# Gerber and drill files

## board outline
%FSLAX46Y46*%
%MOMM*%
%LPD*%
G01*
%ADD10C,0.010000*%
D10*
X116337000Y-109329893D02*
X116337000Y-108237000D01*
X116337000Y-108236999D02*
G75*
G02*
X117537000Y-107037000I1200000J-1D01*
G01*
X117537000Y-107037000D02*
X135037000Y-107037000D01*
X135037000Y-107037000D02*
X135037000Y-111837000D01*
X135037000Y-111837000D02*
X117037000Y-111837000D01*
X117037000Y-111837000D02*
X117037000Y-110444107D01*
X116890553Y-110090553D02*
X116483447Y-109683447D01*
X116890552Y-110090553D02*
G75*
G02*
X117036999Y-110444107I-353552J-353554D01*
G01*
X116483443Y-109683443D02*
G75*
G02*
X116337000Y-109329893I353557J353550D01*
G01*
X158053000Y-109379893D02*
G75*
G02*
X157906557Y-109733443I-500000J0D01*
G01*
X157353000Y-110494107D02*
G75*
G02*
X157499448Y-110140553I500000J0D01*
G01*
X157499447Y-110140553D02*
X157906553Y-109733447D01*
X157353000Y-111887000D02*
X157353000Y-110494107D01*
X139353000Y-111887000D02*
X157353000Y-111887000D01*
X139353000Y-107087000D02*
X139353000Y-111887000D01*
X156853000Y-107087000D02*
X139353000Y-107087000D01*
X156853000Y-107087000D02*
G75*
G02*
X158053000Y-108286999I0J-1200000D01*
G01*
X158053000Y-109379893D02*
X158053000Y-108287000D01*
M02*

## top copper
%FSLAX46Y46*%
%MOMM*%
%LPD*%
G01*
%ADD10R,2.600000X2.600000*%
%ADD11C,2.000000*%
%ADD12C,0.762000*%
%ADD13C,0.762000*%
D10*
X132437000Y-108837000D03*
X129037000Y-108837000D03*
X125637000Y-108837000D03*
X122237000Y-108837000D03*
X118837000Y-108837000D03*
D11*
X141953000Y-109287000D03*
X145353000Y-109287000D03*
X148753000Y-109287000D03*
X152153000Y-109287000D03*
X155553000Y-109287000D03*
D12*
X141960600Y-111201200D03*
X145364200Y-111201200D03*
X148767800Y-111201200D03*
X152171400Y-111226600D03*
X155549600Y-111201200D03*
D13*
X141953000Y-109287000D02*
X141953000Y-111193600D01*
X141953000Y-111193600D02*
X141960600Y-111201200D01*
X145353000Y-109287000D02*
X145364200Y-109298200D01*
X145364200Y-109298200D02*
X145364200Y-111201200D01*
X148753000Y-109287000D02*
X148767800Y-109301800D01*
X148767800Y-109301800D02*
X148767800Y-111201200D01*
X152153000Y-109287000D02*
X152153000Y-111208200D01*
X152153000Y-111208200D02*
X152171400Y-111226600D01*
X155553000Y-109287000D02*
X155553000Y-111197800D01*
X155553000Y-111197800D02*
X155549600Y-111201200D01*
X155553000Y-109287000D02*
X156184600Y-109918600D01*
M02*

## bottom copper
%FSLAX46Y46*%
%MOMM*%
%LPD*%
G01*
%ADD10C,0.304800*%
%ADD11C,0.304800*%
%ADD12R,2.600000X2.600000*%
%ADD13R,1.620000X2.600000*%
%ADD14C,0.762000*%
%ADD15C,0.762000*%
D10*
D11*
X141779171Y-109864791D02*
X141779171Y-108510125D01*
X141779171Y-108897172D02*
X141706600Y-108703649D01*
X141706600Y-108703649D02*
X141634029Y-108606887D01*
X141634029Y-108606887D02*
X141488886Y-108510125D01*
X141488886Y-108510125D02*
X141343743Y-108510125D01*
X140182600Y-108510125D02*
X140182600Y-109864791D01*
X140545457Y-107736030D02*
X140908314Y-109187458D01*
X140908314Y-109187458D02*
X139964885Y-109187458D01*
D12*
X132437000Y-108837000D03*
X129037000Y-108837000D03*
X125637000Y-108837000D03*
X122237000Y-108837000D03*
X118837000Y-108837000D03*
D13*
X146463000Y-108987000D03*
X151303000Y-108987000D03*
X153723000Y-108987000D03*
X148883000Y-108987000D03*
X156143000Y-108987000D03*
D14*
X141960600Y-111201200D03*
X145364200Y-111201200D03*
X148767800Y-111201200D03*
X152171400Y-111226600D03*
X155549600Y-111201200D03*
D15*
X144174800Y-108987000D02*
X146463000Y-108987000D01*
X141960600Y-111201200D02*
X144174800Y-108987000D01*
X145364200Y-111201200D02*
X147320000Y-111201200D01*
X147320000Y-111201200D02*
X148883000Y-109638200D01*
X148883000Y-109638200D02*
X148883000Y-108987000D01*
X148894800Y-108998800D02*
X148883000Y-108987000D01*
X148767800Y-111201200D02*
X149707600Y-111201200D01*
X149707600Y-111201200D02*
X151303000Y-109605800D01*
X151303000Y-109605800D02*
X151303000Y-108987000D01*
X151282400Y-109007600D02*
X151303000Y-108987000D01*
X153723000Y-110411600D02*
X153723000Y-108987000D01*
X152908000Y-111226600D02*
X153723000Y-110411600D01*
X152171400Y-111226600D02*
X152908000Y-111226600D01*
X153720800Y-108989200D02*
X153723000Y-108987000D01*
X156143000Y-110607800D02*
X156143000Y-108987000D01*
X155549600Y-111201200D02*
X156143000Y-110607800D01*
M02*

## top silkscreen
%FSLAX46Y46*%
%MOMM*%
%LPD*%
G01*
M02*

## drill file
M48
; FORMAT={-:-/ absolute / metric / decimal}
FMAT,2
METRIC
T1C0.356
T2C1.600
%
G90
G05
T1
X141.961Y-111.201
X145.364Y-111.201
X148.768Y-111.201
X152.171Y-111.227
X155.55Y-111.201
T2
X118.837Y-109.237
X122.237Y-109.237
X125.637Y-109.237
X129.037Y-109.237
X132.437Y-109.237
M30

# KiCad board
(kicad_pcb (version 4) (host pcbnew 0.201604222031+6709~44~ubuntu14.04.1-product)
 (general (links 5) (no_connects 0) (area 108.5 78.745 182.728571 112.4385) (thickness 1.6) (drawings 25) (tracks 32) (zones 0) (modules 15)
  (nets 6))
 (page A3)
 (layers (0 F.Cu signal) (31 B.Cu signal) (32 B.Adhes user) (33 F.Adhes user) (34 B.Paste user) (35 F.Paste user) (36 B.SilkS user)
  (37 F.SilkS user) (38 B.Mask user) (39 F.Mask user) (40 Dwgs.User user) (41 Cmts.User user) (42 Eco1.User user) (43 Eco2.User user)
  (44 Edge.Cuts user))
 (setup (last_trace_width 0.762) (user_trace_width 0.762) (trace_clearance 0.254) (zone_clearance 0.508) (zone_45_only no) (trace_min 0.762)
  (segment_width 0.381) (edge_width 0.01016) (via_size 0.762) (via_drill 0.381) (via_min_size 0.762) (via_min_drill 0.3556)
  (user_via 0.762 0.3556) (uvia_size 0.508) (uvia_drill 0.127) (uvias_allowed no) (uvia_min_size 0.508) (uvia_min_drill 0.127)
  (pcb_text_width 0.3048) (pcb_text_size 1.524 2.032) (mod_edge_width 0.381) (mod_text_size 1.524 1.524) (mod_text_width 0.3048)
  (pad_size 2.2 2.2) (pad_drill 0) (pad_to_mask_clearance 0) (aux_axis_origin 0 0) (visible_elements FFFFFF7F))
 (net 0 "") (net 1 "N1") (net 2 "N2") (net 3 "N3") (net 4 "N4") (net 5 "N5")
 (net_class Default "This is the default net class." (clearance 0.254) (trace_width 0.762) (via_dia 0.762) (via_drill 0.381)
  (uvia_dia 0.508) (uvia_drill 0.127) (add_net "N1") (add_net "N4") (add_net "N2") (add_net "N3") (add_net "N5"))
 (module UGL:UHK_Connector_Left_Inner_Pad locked (layer B.Cu) (at 132.437 109.237 180)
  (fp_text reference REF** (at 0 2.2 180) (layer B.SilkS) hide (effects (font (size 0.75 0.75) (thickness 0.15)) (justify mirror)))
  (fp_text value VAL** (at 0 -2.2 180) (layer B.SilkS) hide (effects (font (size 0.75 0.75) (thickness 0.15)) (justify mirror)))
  (pad "" thru_hole rect (at 0 0 180) (size 2.6 2.6) (drill 1.6 (offset 0 0.4)) (layers *.Cu *.Mask B.SilkS)))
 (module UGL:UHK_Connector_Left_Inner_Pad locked (layer B.Cu) (at 129.037 109.237 180)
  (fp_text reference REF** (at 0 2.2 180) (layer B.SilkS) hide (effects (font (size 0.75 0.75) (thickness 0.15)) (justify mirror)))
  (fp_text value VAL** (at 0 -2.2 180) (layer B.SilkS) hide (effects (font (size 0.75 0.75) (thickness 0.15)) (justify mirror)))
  (pad "" thru_hole rect (at 0 0 180) (size 2.6 2.6) (drill 1.6 (offset 0 0.4)) (layers *.Cu *.Mask B.SilkS)))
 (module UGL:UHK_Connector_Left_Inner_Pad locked (layer B.Cu) (at 125.637 109.237 180)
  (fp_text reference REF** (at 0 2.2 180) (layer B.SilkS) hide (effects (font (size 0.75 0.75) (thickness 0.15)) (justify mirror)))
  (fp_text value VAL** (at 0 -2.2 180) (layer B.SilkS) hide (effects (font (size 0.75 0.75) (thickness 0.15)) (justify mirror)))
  (pad "" thru_hole rect (at 0 0 180) (size 2.6 2.6) (drill 1.6 (offset 0 0.4)) (layers *.Cu *.Mask B.SilkS)))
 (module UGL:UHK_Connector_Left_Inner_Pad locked (layer B.Cu) (at 122.237 109.237 180)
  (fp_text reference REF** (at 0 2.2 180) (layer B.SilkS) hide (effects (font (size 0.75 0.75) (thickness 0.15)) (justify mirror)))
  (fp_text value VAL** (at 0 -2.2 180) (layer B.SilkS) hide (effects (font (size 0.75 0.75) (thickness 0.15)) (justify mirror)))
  (pad "" thru_hole rect (at 0 0 180) (size 2.6 2.6) (drill 1.6 (offset 0 0.4)) (layers *.Cu *.Mask B.SilkS)))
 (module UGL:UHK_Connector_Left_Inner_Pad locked (layer B.Cu) (at 118.837 109.237 180)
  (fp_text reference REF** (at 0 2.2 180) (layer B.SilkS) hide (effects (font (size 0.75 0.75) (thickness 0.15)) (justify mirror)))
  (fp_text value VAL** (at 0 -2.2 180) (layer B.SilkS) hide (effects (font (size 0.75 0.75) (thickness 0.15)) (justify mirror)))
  (pad "" thru_hole rect (at 0 0 180) (size 2.6 2.6) (drill 1.6 (offset 0 0.4)) (layers *.Cu *.Mask B.SilkS)))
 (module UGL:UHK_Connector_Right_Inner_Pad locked (layer B.Cu) (at 146.463 108.987)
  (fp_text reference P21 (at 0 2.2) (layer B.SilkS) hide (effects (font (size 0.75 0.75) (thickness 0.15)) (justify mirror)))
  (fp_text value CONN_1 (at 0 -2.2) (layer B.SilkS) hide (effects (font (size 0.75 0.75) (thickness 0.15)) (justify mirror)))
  (pad 1 smd rect (at 0 0) (size 1.62 2.6) (layers B.Cu B.Paste B.Mask) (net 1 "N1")))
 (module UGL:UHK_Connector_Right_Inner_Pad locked (layer B.Cu) (at 151.303 108.987)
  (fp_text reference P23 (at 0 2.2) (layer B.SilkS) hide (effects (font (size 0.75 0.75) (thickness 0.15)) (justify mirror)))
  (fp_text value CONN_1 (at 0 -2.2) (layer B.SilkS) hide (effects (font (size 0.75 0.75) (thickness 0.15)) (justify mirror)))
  (pad 1 smd rect (at 0 0) (size 1.62 2.6) (layers B.Cu B.Paste B.Mask) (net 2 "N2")))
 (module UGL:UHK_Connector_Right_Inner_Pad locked (layer B.Cu) (at 153.723 108.987)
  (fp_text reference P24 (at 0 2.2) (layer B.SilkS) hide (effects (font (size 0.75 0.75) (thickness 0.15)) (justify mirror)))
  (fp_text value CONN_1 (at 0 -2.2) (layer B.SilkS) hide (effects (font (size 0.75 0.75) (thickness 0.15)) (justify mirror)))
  (pad 1 smd rect (at 0 0) (size 1.62 2.6) (layers B.Cu B.Paste B.Mask) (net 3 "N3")))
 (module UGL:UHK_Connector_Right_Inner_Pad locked (layer B.Cu) (at 148.883 108.987)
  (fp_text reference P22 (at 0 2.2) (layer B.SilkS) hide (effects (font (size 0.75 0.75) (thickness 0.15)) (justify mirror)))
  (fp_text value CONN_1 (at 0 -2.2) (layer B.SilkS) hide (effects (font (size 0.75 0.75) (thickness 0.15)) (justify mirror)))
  (pad 1 smd rect (at 0 0) (size 1.62 2.6) (layers B.Cu B.Paste B.Mask) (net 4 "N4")))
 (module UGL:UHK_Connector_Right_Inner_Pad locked (layer B.Cu) (at 156.143 108.987)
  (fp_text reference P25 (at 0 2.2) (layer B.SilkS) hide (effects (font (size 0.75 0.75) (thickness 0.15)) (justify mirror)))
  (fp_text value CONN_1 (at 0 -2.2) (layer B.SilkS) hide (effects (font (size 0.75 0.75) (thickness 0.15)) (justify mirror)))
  (pad 1 smd rect (at 0 0) (size 1.62 2.6) (layers B.Cu B.Paste B.Mask) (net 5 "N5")))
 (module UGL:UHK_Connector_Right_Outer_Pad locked (layer F.Cu) (at 141.953 109.287)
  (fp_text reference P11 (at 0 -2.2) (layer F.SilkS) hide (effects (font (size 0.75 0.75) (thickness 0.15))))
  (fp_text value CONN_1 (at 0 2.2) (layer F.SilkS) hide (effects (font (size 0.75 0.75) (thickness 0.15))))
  (pad 1 smd circle (at 0 0) (size 2 2) (layers F.Cu F.Mask) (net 1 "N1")))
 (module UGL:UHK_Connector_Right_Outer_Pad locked (layer F.Cu) (at 145.353 109.287)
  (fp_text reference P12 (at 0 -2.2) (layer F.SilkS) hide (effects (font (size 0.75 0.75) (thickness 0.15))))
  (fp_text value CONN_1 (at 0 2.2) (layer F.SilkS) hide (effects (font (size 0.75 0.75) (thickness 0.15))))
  (pad 1 smd circle (at 0 0) (size 2 2) (layers F.Cu F.Mask) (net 4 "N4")))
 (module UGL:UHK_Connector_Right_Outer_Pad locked (layer F.Cu) (at 148.753 109.287)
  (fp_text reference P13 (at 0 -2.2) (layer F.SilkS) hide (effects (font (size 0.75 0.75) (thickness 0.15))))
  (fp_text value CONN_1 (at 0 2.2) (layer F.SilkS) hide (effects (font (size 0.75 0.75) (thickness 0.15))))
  (pad 1 smd circle (at 0 0) (size 2 2) (layers F.Cu F.Mask) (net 2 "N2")))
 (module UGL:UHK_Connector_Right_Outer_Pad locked (layer F.Cu) (at 152.153 109.287)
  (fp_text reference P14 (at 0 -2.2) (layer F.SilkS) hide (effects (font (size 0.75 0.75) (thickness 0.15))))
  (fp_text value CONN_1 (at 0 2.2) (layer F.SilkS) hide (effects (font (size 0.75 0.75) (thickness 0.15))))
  (pad 1 smd circle (at 0 0) (size 2 2) (layers F.Cu F.Mask) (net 3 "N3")))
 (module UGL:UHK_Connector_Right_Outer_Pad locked (layer F.Cu) (at 155.553 109.287)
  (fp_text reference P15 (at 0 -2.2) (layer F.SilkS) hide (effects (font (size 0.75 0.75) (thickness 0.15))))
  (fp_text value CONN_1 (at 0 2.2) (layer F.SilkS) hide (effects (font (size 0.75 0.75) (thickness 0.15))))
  (pad 1 smd circle (at 0 0) (size 2 2) (layers F.Cu F.Mask) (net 5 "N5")))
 (gr_line (start 116.337 109.329893) (end 116.337 108.237) (angle 90) (layer Edge.Cuts) (width 0.01))
 (gr_arc (start 117.537 108.237) (end 117.537 107.037) (angle -89.99995347) (layer Edge.Cuts) (width 0.01))
 (gr_line (start 117.537 107.037) (end 135.037 107.037) (angle 90) (layer Edge.Cuts) (width 0.01))
 (gr_line (start 135.037 107.037) (end 135.037 111.837) (angle 90) (layer Edge.Cuts) (width 0.01))
 (gr_line (start 135.037 111.837) (end 117.037 111.837) (angle 90) (layer Edge.Cuts) (width 0.01))
 (gr_line (start 117.037 111.837) (end 117.037 110.444107) (angle 90) (layer Edge.Cuts) (width 0.01))
 (gr_line (start 116.890553 110.090553) (end 116.483447 109.683447) (angle 90) (layer Edge.Cuts) (width 0.01))
 (gr_arc (start 116.537 110.444107) (end 117.037 110.444107) (angle -45.00015451) (layer Edge.Cuts) (width 0.01))
 (gr_arc (start 116.837 109.329893) (end 116.337 109.329893) (angle -44.99944414) (layer Edge.Cuts) (width 0.01))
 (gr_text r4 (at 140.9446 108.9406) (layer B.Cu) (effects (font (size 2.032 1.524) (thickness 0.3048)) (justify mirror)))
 (gr_arc (start 157.553 109.379893) (end 158.053 109.379893) (angle 44.99944414) (layer Edge.Cuts) (width 0.01))
 (gr_arc (start 157.853 110.494107) (end 157.353 110.494107) (angle 45.00015451) (layer Edge.Cuts) (width 0.01))
 (gr_line (start 157.499447 110.140553) (end 157.906553 109.733447) (angle 90) (layer Edge.Cuts) (width 0.01))
 (gr_line (start 157.353 111.887) (end 157.353 110.494107) (angle 90) (layer Edge.Cuts) (width 0.01))
 (gr_line (start 139.353 111.887) (end 157.353 111.887) (angle 90) (layer Edge.Cuts) (width 0.01))
 (gr_line (start 139.353 107.087) (end 139.353 111.887) (angle 90) (layer Edge.Cuts) (width 0.01))
 (gr_line (start 156.853 107.087) (end 139.353 107.087) (angle 90) (layer Edge.Cuts) (width 0.01))
 (gr_arc (start 156.853 108.287) (end 156.853 107.087) (angle 89.99995347) (layer Edge.Cuts) (width 0.01))
 (gr_line (start 158.053 109.379893) (end 158.053 108.287) (angle 90) (layer Edge.Cuts) (width 0.01))
 (segment (start 141.953 109.287) (end 141.953 111.1936) (width 0.762) (layer F.Cu) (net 1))
 (segment (start 144.1748 108.987) (end 146.463 108.987) (width 0.762) (layer B.Cu) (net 1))
 (segment (start 141.9606 111.2012) (end 144.1748 108.987) (width 0.762) (layer B.Cu) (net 1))
 (via (at 141.9606 111.2012) (size 0.762) (drill 0.3556) (layers F.Cu B.Cu) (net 1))
 (segment (start 141.953 111.1936) (end 141.9606 111.2012) (width 0.762) (layer F.Cu) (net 1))
 (segment (start 145.353 109.287) (end 145.3642 109.2982) (width 0.762) (layer F.Cu) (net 4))
 (segment (start 145.3642 109.2982) (end 145.3642 111.2012) (width 0.762) (layer F.Cu) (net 4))
 (via (at 145.3642 111.2012) (size 0.762) (drill 0.3556) (layers F.Cu B.Cu) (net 4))
 (segment (start 145.3642 111.2012) (end 147.32 111.2012) (width 0.762) (layer B.Cu) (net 4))
 (segment (start 147.32 111.2012) (end 148.883 109.6382) (width 0.762) (layer B.Cu) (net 4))
 (segment (start 148.883 109.6382) (end 148.883 108.987) (width 0.762) (layer B.Cu) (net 4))
 (segment (start 148.8948 108.9988) (end 148.883 108.987) (width 0.762) (layer B.Cu) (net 4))
 (segment (start 148.753 109.287) (end 148.7678 109.3018) (width 0.762) (layer F.Cu) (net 2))
 (segment (start 148.7678 109.3018) (end 148.7678 111.2012) (width 0.762) (layer F.Cu) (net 2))
 (via (at 148.7678 111.2012) (size 0.762) (drill 0.3556) (layers F.Cu B.Cu) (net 2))
 (segment (start 148.7678 111.2012) (end 149.7076 111.2012) (width 0.762) (layer B.Cu) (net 2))
 (segment (start 149.7076 111.2012) (end 151.303 109.6058) (width 0.762) (layer B.Cu) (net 2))
 (segment (start 151.303 109.6058) (end 151.303 108.987) (width 0.762) (layer B.Cu) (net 2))
 (segment (start 151.2824 109.0076) (end 151.303 108.987) (width 0.762) (layer B.Cu) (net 2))
 (segment (start 152.153 109.287) (end 152.153 111.2082) (width 0.762) (layer F.Cu) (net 3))
 (segment (start 153.723 110.4116) (end 153.723 108.987) (width 0.762) (layer B.Cu) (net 3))
 (segment (start 152.908 111.2266) (end 153.723 110.4116) (width 0.762) (layer B.Cu) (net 3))
 (segment (start 152.1714 111.2266) (end 152.908 111.2266) (width 0.762) (layer B.Cu) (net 3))
 (via (at 152.1714 111.2266) (size 0.762) (drill 0.3556) (layers F.Cu B.Cu) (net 3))
 (segment (start 152.153 111.2082) (end 152.1714 111.2266) (width 0.762) (layer F.Cu) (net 3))
 (segment (start 153.7208 108.9892) (end 153.723 108.987) (width 0.762) (layer B.Cu) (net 3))
 (segment (start 155.553 109.287) (end 155.553 111.1978) (width 0.762) (layer F.Cu) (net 5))
 (segment (start 156.143 110.6078) (end 156.143 108.987) (width 0.762) (layer B.Cu) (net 5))
 (segment (start 155.5496 111.2012) (end 156.143 110.6078) (width 0.762) (layer B.Cu) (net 5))
 (via (at 155.5496 111.2012) (size 0.762) (drill 0.3556) (layers F.Cu B.Cu) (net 5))
 (segment (start 155.553 111.1978) (end 155.5496 111.2012) (width 0.762) (layer F.Cu) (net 5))
 (segment (start 155.553 109.287) (end 156.1846 109.9186) (width 0.762) (layer F.Cu) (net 5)))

